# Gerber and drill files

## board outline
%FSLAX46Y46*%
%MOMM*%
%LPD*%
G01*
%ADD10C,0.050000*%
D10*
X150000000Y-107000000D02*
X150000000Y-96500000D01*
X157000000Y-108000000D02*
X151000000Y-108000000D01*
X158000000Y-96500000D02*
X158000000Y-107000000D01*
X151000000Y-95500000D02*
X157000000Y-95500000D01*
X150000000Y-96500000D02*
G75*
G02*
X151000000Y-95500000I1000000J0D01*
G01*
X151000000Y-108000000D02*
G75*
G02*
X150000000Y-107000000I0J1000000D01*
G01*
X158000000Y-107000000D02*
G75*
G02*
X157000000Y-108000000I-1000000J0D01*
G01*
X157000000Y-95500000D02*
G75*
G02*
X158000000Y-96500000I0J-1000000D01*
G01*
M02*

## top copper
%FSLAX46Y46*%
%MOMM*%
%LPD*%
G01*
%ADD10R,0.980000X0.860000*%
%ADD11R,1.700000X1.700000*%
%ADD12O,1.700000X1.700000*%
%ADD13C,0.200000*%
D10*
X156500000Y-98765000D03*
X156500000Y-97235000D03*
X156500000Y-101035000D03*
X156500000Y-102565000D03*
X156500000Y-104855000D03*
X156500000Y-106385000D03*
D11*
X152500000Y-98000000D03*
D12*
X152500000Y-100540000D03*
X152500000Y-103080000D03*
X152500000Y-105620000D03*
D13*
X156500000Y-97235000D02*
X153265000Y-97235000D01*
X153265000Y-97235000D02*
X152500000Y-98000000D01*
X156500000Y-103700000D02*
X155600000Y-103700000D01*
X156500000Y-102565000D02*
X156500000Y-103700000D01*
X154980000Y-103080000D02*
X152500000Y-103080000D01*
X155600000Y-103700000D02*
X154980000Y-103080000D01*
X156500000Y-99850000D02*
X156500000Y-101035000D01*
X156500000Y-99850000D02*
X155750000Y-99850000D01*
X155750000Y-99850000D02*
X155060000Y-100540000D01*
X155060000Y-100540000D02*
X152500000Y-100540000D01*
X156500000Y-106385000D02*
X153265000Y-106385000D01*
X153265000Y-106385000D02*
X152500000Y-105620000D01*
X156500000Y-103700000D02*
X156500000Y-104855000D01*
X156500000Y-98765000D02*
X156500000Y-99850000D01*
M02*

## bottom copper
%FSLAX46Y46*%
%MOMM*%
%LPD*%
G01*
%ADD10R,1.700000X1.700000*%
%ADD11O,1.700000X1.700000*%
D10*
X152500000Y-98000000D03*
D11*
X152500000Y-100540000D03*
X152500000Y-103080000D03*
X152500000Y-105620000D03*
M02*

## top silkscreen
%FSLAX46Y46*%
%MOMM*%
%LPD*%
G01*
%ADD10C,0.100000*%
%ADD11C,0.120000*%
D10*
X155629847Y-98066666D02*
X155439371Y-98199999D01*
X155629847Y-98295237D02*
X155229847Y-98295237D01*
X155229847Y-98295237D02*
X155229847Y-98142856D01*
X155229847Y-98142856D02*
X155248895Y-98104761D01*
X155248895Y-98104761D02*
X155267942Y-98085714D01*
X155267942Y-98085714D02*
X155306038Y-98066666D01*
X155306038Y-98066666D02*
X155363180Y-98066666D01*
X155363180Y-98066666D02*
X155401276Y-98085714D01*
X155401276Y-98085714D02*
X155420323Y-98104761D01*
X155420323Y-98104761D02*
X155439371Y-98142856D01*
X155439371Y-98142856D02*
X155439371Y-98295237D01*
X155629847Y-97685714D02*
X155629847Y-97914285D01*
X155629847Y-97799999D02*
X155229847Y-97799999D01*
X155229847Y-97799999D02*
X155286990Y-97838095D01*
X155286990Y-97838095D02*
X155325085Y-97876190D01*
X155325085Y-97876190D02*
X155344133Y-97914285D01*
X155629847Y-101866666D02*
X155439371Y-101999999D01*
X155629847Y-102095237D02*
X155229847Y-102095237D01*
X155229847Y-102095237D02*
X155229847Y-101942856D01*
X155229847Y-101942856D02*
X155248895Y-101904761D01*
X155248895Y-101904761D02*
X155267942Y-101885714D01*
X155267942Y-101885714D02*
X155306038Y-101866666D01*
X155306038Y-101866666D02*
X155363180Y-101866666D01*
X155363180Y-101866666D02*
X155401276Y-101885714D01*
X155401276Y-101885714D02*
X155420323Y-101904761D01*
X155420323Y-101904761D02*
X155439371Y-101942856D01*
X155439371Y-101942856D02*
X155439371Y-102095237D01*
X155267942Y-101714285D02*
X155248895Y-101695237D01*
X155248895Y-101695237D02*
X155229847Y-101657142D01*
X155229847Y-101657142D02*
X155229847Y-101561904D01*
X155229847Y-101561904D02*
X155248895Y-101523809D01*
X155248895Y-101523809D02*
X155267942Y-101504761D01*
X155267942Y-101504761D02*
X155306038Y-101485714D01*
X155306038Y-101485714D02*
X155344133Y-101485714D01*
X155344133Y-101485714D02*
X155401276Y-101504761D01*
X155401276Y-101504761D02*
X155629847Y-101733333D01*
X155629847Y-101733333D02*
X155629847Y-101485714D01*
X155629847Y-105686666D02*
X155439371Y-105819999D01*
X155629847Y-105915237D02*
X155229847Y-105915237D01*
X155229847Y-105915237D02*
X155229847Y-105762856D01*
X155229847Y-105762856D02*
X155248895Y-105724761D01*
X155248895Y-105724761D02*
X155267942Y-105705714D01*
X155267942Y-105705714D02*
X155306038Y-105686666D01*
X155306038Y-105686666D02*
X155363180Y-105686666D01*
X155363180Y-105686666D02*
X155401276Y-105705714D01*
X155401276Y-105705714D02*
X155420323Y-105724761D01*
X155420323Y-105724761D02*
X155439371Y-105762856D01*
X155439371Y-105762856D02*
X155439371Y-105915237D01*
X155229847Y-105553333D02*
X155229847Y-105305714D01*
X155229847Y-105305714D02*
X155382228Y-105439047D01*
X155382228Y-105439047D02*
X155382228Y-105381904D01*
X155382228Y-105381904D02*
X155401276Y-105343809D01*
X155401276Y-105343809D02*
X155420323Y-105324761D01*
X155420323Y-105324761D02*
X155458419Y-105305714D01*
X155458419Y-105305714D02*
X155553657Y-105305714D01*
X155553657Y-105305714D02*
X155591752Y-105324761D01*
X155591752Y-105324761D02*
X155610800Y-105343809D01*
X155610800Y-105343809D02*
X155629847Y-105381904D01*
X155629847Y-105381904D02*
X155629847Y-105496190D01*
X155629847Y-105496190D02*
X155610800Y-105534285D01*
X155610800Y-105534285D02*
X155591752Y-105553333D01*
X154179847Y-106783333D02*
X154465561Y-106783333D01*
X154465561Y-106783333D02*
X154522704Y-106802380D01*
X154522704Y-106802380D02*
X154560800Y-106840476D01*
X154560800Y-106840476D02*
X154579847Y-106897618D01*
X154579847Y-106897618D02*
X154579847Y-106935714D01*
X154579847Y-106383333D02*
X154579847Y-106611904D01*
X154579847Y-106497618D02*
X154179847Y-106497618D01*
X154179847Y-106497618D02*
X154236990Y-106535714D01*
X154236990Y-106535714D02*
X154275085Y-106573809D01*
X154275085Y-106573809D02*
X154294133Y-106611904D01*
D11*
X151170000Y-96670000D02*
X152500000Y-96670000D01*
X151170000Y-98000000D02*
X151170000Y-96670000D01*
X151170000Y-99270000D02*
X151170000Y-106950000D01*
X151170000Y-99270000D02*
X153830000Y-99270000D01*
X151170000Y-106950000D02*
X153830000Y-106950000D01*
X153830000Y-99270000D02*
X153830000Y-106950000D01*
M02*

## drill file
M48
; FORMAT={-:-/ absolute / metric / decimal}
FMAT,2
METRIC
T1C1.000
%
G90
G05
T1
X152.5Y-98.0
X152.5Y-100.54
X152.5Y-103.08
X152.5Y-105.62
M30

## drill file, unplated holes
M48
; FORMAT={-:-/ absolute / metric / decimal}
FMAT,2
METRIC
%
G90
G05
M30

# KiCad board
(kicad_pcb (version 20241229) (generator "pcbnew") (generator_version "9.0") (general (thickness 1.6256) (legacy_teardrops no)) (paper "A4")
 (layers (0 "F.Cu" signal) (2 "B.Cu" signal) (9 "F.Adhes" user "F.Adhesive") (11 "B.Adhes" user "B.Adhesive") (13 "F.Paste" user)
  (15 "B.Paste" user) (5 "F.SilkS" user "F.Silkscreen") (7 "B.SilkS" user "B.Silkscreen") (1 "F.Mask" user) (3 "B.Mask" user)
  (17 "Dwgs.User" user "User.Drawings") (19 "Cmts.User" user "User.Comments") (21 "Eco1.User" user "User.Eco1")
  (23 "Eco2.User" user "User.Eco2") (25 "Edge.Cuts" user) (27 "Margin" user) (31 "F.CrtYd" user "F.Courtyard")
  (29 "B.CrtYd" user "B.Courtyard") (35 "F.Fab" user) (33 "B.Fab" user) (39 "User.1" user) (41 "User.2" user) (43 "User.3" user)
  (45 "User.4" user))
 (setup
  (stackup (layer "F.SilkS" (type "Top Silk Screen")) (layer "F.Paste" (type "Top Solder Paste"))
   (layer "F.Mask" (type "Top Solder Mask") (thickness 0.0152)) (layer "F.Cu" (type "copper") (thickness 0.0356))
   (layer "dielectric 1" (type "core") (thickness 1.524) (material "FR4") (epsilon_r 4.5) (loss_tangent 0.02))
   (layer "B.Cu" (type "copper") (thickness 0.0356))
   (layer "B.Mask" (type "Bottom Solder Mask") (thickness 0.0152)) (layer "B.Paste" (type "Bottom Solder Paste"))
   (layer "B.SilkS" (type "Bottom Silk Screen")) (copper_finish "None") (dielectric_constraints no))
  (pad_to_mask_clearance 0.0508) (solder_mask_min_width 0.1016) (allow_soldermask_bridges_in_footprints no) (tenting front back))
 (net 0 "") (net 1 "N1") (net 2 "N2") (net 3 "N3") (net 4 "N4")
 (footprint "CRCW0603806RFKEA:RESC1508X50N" (layer "F.Cu") (at 156.5 101.8 -90)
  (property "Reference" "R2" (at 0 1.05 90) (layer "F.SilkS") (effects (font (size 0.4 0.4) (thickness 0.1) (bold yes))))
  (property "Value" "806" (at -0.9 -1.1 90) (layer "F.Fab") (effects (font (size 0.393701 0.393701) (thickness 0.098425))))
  (pad "1" smd rect (at -0.765 0 270) (size 0.86 0.98) (layers "F.Cu" "F.Mask" "F.Paste") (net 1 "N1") (solder_mask_margin 0.102))
  (pad "2" smd rect (at 0.765 0 270) (size 0.86 0.98) (layers "F.Cu" "F.Mask" "F.Paste") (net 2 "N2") (solder_mask_margin 0.102)))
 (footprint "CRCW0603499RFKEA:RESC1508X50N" (layer "F.Cu") (at 156.5 105.62 -90)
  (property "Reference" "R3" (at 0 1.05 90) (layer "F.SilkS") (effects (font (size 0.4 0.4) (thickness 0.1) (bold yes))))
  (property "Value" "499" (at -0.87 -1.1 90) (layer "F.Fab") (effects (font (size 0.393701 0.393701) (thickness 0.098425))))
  (pad "1" smd rect (at -0.765 0 270) (size 0.86 0.98) (layers "F.Cu" "F.Mask" "F.Paste") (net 2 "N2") (solder_mask_margin 0.102))
  (pad "2" smd rect (at 0.765 0 270) (size 0.86 0.98) (layers "F.Cu" "F.Mask" "F.Paste") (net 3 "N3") (solder_mask_margin 0.102)))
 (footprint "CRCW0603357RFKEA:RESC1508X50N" (layer "F.Cu") (at 156.5 98 -90)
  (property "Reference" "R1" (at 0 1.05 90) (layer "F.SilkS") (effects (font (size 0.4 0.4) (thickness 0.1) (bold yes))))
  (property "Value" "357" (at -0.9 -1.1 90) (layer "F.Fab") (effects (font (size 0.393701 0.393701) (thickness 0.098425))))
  (pad "1" smd rect (at -0.765 0 270) (size 0.86 0.98) (layers "F.Cu" "F.Mask" "F.Paste") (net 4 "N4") (solder_mask_margin 0.102))
  (pad "2" smd rect (at 0.765 0 270) (size 0.86 0.98) (layers "F.Cu" "F.Mask" "F.Paste") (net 1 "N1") (solder_mask_margin 0.102)))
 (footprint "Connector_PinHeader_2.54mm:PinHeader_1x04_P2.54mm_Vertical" (layer "F.Cu") (at 152.5 98)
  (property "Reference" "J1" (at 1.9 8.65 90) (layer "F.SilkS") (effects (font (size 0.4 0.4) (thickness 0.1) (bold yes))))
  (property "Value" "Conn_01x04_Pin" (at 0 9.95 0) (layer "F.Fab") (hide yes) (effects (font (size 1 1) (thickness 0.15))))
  (fp_line (start -1.33 -1.33) (end 0 -1.33) (stroke (width 0.12) (type solid)) (layer "F.SilkS"))
  (fp_line (start -1.33 0) (end -1.33 -1.33) (stroke (width 0.12) (type solid)) (layer "F.SilkS"))
  (fp_line (start -1.33 1.27) (end -1.33 8.95) (stroke (width 0.12) (type solid)) (layer "F.SilkS"))
  (fp_line (start -1.33 1.27) (end 1.33 1.27) (stroke (width 0.12) (type solid)) (layer "F.SilkS"))
  (fp_line (start -1.33 8.95) (end 1.33 8.95) (stroke (width 0.12) (type solid)) (layer "F.SilkS"))
  (fp_line (start 1.33 1.27) (end 1.33 8.95) (stroke (width 0.12) (type solid)) (layer "F.SilkS"))
  (pad "1" thru_hole rect (at 0 0) (size 1.7 1.7) (drill 1) (layers "*.Cu" "*.Mask") (remove_unused_layers no) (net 4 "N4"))
  (pad "2" thru_hole oval (at 0 2.54) (size 1.7 1.7) (drill 1) (layers "*.Cu" "*.Mask") (remove_unused_layers no) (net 1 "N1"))
  (pad "3" thru_hole oval (at 0 5.08) (size 1.7 1.7) (drill 1) (layers "*.Cu" "*.Mask") (remove_unused_layers no) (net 2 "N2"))
  (pad "4" thru_hole oval (at 0 7.62) (size 1.7 1.7) (drill 1) (layers "*.Cu" "*.Mask") (remove_unused_layers no) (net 3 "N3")))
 (gr_arc (start 157 95.5) (mid 157.707107 95.792893) (end 158 96.5) (stroke (width 0.05) (type default)) (layer "Edge.Cuts"))
 (gr_arc (start 150 96.5) (mid 150.292893 95.792893) (end 151 95.5) (stroke (width 0.05) (type default)) (layer "Edge.Cuts"))
 (gr_line (start 150 107) (end 150 96.5) (stroke (width 0.05) (type default)) (layer "Edge.Cuts"))
 (gr_line (start 158 96.5) (end 158 107) (stroke (width 0.05) (type default)) (layer "Edge.Cuts"))
 (gr_line (start 151 95.5) (end 157 95.5) (stroke (width 0.05) (type default)) (layer "Edge.Cuts"))
 (gr_line (start 157 108) (end 151 108) (stroke (width 0.05) (type default)) (layer "Edge.Cuts"))
 (gr_arc (start 158 107) (mid 157.707107 107.707107) (end 157 108) (stroke (width 0.05) (type default)) (layer "Edge.Cuts"))
 (gr_arc (start 151 108) (mid 150.292893 107.707107) (end 150 107) (stroke (width 0.05) (type default)) (layer "Edge.Cuts"))
 (segment (start 153.265 106.385) (end 152.5 105.62) (width 0.2) (layer "F.Cu") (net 3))
 (segment (start 156.5 106.385) (end 153.265 106.385) (width 0.2) (layer "F.Cu") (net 3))
 (segment (start 156.5 97.235) (end 153.265 97.235) (width 0.2) (layer "F.Cu") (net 4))
 (segment (start 153.265 97.235) (end 152.5 98) (width 0.2) (layer "F.Cu") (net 4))
 (segment (start 155.06 100.54) (end 152.5 100.54) (width 0.2) (layer "F.Cu") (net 1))
 (segment (start 156.5 99.85) (end 155.75 99.85) (width 0.2) (layer "F.Cu") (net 1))
 (segment (start 155.75 99.85) (end 155.06 100.54) (width 0.2) (layer "F.Cu") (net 1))
 (segment (start 156.5 98.765) (end 156.5 99.85) (width 0.2) (layer "F.Cu") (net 1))
 (segment (start 156.5 99.85) (end 156.5 101.035) (width 0.2) (layer "F.Cu") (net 1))
 (segment (start 156.5 102.565) (end 156.5 103.7) (width 0.2) (layer "F.Cu") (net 2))
 (segment (start 154.98 103.08) (end 152.5 103.08) (width 0.2) (layer "F.Cu") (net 2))
 (segment (start 156.5 103.7) (end 155.6 103.7) (width 0.2) (layer "F.Cu") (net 2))
 (segment (start 155.6 103.7) (end 154.98 103.08) (width 0.2) (layer "F.Cu") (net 2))
 (segment (start 156.5 103.7) (end 156.5 104.855) (width 0.2) (layer "F.Cu") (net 2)))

